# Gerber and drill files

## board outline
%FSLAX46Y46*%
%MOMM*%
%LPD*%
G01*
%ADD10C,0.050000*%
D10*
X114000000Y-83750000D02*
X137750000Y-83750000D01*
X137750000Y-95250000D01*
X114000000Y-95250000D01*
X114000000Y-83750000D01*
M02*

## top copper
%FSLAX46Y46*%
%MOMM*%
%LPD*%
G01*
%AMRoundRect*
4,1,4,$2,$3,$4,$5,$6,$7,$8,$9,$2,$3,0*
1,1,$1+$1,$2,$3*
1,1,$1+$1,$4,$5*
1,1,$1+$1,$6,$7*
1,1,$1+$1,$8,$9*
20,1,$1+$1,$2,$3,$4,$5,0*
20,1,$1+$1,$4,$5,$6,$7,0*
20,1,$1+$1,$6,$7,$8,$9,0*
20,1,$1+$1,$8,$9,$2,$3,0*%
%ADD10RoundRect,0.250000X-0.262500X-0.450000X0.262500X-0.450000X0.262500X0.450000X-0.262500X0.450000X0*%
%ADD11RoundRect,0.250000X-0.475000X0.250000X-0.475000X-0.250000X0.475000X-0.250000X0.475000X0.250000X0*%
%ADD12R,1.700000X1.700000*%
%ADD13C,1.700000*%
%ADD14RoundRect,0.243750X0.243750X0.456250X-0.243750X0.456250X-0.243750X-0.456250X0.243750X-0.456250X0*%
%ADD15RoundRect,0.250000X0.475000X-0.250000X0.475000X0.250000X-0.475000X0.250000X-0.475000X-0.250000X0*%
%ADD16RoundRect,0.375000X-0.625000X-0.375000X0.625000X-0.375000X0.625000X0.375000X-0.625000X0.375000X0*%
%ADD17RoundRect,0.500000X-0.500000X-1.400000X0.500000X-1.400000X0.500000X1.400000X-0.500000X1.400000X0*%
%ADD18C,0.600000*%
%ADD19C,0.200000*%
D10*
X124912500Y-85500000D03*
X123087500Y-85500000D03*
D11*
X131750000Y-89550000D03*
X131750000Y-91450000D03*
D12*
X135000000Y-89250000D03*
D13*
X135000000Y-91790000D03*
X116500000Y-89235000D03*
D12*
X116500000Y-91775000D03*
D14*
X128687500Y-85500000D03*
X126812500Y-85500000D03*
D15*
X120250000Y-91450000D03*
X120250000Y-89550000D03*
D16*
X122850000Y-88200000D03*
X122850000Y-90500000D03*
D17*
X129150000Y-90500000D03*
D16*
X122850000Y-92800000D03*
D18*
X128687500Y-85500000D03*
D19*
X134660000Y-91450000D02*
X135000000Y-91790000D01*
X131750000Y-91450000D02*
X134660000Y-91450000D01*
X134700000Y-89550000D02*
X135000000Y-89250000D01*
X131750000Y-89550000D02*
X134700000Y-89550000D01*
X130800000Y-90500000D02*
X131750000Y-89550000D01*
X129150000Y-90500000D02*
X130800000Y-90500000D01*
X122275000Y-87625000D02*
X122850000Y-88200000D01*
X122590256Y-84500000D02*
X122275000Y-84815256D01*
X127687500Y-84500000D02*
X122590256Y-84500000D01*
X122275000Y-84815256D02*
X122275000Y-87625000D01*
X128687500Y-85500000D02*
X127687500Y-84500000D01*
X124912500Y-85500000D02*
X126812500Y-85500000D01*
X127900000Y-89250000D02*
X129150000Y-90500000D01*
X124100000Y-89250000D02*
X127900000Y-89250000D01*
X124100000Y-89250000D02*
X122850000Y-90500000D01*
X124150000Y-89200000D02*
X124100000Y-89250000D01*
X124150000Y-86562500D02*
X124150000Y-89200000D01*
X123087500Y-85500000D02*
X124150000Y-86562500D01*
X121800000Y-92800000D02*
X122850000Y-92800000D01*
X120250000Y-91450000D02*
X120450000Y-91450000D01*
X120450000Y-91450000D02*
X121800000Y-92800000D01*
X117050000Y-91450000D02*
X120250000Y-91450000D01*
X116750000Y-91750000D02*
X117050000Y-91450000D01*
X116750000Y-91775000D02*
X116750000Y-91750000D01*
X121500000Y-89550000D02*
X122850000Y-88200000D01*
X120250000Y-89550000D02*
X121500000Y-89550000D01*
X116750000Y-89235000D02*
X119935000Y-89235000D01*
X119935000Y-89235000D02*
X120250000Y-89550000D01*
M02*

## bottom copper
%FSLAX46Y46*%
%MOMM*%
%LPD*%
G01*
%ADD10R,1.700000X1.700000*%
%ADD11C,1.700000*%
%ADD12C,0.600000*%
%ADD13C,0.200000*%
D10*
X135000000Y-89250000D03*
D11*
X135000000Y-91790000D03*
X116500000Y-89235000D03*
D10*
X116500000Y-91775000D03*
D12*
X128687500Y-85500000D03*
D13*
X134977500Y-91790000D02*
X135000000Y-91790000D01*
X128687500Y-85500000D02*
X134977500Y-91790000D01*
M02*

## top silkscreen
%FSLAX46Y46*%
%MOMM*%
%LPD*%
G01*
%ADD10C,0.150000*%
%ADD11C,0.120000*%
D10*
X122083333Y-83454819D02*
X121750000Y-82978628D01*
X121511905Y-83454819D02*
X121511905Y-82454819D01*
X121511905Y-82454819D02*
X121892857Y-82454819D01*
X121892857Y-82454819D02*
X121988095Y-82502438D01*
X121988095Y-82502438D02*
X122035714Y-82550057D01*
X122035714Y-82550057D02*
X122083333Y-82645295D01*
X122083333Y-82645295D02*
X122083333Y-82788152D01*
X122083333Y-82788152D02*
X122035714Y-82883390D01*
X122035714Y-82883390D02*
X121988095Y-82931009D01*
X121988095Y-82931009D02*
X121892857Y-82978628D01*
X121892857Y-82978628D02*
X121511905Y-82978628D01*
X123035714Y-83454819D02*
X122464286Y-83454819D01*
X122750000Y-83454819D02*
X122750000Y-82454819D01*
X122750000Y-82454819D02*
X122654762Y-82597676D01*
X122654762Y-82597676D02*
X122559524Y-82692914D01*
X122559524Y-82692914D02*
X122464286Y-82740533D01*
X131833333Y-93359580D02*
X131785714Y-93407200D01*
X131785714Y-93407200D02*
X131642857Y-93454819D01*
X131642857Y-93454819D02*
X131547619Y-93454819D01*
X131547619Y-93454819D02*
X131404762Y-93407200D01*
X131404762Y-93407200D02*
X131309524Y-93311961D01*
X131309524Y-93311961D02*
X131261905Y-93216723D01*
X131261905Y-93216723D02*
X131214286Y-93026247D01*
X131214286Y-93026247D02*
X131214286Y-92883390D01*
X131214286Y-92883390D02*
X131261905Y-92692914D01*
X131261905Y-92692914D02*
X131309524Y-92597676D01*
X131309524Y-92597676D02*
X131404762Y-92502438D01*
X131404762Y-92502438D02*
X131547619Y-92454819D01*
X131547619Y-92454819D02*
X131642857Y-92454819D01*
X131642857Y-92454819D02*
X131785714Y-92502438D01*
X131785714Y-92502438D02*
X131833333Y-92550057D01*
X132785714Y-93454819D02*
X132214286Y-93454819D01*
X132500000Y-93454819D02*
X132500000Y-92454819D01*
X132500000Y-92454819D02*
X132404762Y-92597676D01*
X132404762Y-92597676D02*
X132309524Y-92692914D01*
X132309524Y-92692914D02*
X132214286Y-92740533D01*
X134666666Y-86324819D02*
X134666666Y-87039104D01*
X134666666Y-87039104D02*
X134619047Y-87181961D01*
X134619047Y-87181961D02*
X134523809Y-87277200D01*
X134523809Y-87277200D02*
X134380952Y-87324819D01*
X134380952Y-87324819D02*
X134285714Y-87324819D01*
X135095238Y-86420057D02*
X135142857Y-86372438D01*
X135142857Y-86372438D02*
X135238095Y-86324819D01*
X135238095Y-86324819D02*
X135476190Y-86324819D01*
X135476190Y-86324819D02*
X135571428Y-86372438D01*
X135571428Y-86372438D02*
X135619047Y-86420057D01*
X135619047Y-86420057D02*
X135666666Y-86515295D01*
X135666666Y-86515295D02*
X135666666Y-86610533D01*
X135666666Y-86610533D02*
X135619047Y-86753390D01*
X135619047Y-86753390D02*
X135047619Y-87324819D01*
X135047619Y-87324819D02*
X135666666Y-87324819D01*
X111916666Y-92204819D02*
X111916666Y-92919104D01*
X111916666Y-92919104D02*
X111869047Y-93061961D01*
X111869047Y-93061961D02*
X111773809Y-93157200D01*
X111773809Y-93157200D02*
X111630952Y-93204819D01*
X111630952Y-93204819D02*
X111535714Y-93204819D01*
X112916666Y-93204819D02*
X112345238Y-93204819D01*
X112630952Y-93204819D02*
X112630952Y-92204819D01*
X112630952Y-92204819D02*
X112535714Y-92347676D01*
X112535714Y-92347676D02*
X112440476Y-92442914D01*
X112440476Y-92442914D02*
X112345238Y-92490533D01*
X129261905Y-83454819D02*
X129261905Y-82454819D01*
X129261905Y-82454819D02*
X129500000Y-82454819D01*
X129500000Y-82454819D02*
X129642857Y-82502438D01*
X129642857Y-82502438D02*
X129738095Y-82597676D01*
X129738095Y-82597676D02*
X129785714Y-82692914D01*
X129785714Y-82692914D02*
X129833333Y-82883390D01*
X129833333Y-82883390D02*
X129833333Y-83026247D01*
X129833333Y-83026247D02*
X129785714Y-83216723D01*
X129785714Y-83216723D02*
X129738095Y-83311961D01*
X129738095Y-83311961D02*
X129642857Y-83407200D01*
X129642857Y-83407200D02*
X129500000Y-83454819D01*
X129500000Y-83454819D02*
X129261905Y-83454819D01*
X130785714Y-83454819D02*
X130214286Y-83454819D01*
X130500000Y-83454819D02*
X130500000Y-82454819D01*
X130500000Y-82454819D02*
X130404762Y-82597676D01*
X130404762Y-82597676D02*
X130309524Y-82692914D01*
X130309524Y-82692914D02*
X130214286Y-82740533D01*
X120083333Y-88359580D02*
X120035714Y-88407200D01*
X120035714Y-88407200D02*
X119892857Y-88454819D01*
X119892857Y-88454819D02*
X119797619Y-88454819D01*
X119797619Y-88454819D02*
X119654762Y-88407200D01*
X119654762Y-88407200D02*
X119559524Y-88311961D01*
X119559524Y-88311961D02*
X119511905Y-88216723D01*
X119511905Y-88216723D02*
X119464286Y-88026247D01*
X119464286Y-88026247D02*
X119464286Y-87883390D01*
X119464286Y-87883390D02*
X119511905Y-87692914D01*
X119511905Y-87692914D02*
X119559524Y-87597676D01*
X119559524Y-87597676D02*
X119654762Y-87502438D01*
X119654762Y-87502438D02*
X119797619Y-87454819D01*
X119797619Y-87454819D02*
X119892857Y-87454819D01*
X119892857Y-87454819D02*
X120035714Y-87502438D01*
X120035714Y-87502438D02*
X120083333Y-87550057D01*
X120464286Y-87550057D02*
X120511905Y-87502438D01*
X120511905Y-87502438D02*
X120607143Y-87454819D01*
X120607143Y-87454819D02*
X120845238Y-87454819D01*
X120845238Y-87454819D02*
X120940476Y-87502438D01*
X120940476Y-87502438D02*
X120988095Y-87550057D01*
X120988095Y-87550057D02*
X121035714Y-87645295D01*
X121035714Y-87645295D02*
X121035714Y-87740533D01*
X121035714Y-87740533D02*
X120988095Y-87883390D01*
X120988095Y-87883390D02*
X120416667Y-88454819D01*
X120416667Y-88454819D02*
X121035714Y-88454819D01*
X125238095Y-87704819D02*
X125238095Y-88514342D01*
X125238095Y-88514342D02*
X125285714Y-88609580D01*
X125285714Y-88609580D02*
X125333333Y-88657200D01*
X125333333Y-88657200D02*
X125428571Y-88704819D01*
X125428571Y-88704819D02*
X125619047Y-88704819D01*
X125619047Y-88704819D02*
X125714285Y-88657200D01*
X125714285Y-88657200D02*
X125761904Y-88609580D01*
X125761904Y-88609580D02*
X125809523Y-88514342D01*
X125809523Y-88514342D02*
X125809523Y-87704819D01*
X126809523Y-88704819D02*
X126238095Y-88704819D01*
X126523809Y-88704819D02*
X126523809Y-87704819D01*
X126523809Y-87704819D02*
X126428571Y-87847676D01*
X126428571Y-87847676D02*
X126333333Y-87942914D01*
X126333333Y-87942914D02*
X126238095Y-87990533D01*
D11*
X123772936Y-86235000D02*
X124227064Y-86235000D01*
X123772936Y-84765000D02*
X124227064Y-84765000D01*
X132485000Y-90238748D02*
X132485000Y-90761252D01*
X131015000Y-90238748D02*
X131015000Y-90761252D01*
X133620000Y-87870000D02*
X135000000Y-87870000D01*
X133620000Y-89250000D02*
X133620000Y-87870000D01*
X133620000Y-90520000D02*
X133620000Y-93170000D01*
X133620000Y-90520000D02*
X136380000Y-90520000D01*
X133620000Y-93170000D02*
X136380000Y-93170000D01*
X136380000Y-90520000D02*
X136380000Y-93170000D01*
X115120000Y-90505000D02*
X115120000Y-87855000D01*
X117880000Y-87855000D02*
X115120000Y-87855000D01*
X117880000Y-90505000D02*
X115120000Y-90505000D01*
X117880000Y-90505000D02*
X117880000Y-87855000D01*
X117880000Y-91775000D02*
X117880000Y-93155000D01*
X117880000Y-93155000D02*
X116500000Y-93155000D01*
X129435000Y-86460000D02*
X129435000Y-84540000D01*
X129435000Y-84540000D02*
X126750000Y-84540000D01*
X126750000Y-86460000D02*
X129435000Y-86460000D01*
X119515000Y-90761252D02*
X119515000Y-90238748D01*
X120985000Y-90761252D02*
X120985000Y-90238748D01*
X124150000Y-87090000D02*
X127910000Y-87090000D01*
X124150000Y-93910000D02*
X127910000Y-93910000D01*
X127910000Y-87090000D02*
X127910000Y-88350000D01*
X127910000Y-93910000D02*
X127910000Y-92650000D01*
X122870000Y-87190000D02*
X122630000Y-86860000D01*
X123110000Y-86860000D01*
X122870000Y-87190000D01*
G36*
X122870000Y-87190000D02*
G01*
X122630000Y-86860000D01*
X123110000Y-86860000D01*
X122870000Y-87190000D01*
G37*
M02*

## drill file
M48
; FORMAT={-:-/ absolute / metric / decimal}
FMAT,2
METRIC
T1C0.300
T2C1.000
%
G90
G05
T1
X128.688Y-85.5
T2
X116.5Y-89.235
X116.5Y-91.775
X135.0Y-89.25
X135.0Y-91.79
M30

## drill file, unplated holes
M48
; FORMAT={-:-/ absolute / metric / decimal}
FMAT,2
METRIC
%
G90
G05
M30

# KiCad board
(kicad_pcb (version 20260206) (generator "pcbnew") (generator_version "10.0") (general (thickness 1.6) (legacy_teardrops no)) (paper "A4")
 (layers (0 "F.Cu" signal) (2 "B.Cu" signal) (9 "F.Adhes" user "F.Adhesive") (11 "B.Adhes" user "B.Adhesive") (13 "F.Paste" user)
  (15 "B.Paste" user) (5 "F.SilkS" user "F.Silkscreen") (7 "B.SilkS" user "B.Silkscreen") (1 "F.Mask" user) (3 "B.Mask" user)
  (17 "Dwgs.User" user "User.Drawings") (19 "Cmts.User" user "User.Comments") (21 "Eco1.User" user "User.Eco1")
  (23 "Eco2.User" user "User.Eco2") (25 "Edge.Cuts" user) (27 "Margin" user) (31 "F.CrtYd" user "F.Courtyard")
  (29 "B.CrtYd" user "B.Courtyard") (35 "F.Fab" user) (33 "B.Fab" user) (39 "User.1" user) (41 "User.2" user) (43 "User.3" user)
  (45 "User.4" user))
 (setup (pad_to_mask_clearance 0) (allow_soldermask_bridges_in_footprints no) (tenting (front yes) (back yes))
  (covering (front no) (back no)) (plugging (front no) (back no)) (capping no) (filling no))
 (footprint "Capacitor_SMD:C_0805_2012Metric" (layer "F.Cu") (at 131.75 90.5 -90)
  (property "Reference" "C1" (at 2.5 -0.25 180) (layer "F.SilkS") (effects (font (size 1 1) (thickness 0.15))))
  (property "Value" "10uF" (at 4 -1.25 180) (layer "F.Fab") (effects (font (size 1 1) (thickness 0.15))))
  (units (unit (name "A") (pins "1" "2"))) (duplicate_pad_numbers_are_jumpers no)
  (fp_line (start -0.261252 0.735) (end 0.261252 0.735) (stroke (width 0.12) (type solid)) (layer "F.SilkS"))
  (fp_line (start -0.261252 -0.735) (end 0.261252 -0.735) (stroke (width 0.12) (type solid)) (layer "F.SilkS"))
  (pad "1" smd roundrect (at -0.95 0 270) (size 1 1.45) (layers "F.Cu" "F.Mask" "F.Paste") (roundrect_rratio 0.25) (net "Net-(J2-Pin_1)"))
  (pad "2" smd roundrect (at 0.95 0 270) (size 1 1.45) (layers "F.Cu" "F.Mask" "F.Paste") (roundrect_rratio 0.25) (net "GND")))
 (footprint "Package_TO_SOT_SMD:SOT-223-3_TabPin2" (layer "F.Cu") (at 126 90.5)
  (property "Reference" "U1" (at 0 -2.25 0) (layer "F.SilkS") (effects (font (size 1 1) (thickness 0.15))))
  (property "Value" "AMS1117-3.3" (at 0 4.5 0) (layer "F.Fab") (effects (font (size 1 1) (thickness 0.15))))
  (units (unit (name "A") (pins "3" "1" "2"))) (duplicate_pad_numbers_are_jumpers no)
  (fp_line (start -1.85 -3.41) (end 1.91 -3.41) (stroke (width 0.12) (type solid)) (layer "F.SilkS"))
  (fp_line (start -1.85 3.41) (end 1.91 3.41) (stroke (width 0.12) (type solid)) (layer "F.SilkS"))
  (fp_line (start 1.91 -3.41) (end 1.91 -2.15) (stroke (width 0.12) (type solid)) (layer "F.SilkS"))
  (fp_line (start 1.91 3.41) (end 1.91 2.15) (stroke (width 0.12) (type solid)) (layer "F.SilkS"))
  (fp_poly
   (pts (xy -3.13 -3.31) (xy -3.37 -3.64) (xy -2.89 -3.64) (xy -3.13 -3.31)) (stroke (width 0.12) (type solid)) (fill yes) (layer "F.SilkS"))
  (pad "1" smd roundrect (at -3.15 -2.3) (size 2 1.5) (layers "F.Cu" "F.Mask" "F.Paste") (roundrect_rratio 0.25) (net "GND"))
  (pad "2" smd roundrect (at -3.15 0) (size 2 1.5) (layers "F.Cu" "F.Mask" "F.Paste") (roundrect_rratio 0.25) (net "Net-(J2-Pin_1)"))
  (pad "2" smd roundrect (at 3.15 0) (size 2 3.8) (layers "F.Cu" "F.Mask" "F.Paste") (roundrect_rratio 0.25) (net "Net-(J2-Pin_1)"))
  (pad "3" smd roundrect (at -3.15 2.3) (size 2 1.5) (layers "F.Cu" "F.Mask" "F.Paste") (roundrect_rratio 0.25) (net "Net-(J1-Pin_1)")))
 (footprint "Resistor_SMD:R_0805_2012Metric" (layer "F.Cu") (at 124 85.5)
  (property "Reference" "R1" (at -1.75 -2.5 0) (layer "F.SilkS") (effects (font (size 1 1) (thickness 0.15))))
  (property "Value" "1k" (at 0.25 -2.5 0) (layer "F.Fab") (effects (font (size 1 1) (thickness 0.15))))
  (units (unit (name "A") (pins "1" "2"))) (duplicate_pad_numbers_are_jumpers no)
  (fp_line (start -0.227064 -0.735) (end 0.227064 -0.735) (stroke (width 0.12) (type solid)) (layer "F.SilkS"))
  (fp_line (start -0.227064 0.735) (end 0.227064 0.735) (stroke (width 0.12) (type solid)) (layer "F.SilkS"))
  (pad "1" smd roundrect (at -0.9125 0) (size 1.025 1.4) (layers "F.Cu" "F.Mask" "F.Paste") (roundrect_rratio 0.243902)
   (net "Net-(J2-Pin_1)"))
  (pad "2" smd roundrect (at 0.9125 0) (size 1.025 1.4) (layers "F.Cu" "F.Mask" "F.Paste") (roundrect_rratio 0.243902) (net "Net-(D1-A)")))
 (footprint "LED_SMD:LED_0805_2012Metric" (layer "F.Cu") (at 127.75 85.5 180)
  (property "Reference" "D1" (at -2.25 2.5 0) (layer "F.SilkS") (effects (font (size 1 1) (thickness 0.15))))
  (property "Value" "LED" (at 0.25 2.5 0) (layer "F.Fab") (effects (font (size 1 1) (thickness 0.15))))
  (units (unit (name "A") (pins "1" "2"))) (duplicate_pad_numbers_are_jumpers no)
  (fp_line (start 1 -0.96) (end -1.685 -0.96) (stroke (width 0.12) (type solid)) (layer "F.SilkS"))
  (fp_line (start -1.685 0.96) (end 1 0.96) (stroke (width 0.12) (type solid)) (layer "F.SilkS"))
  (fp_line (start -1.685 -0.96) (end -1.685 0.96) (stroke (width 0.12) (type solid)) (layer "F.SilkS"))
  (pad "1" smd roundrect (at -0.9375 0 180) (size 0.975 1.4) (layers "F.Cu" "F.Mask" "F.Paste") (roundrect_rratio 0.25) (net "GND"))
  (pad "2" smd roundrect (at 0.9375 0 180) (size 0.975 1.4) (layers "F.Cu" "F.Mask" "F.Paste") (roundrect_rratio 0.25) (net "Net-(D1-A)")))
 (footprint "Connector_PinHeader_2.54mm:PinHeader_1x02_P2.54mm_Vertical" (layer "F.Cu") (at 116.5 91.775 180)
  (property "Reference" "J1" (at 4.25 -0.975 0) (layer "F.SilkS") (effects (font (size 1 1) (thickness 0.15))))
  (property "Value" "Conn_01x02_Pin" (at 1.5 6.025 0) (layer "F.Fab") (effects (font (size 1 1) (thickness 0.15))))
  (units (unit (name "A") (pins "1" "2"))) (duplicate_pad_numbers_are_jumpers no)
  (fp_line (start 1.38 1.27) (end 1.38 3.92) (stroke (width 0.12) (type solid)) (layer "F.SilkS"))
  (fp_line (start -1.38 3.92) (end 1.38 3.92) (stroke (width 0.12) (type solid)) (layer "F.SilkS"))
  (fp_line (start -1.38 1.27) (end 1.38 1.27) (stroke (width 0.12) (type solid)) (layer "F.SilkS"))
  (fp_line (start -1.38 1.27) (end -1.38 3.92) (stroke (width 0.12) (type solid)) (layer "F.SilkS"))
  (fp_line (start -1.38 0) (end -1.38 -1.38) (stroke (width 0.12) (type solid)) (layer "F.SilkS"))
  (fp_line (start -1.38 -1.38) (end 0 -1.38) (stroke (width 0.12) (type solid)) (layer "F.SilkS"))
  (pad "1" thru_hole rect (at 0 0 180) (size 1.7 1.7) (drill 1) (layers "*.Cu" "*.Mask") (remove_unused_layers no) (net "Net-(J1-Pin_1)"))
  (pad "2" thru_hole circle (at 0 2.54 180) (size 1.7 1.7) (drill 1) (layers "*.Cu" "*.Mask") (remove_unused_layers no) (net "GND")))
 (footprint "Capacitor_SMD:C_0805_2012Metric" (layer "F.Cu") (at 120.25 90.5 90)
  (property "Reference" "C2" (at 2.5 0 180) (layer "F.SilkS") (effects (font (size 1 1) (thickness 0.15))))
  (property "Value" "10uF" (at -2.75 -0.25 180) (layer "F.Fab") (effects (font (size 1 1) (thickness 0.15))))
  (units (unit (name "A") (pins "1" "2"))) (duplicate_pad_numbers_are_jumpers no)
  (fp_line (start -0.261252 -0.735) (end 0.261252 -0.735) (stroke (width 0.12) (type solid)) (layer "F.SilkS"))
  (fp_line (start -0.261252 0.735) (end 0.261252 0.735) (stroke (width 0.12) (type solid)) (layer "F.SilkS"))
  (pad "1" smd roundrect (at -0.95 0 90) (size 1 1.45) (layers "F.Cu" "F.Mask" "F.Paste") (roundrect_rratio 0.25) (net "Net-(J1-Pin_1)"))
  (pad "2" smd roundrect (at 0.95 0 90) (size 1 1.45) (layers "F.Cu" "F.Mask" "F.Paste") (roundrect_rratio 0.25) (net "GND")))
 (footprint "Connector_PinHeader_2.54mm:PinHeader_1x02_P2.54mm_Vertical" (layer "F.Cu") (at 135 89.25)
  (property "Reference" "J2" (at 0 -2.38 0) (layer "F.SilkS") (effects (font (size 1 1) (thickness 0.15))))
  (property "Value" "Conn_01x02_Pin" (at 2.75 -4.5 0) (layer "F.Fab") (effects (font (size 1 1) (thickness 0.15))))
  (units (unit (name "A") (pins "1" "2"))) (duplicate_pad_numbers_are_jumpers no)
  (fp_line (start -1.38 -1.38) (end 0 -1.38) (stroke (width 0.12) (type solid)) (layer "F.SilkS"))
  (fp_line (start -1.38 0) (end -1.38 -1.38) (stroke (width 0.12) (type solid)) (layer "F.SilkS"))
  (fp_line (start -1.38 1.27) (end -1.38 3.92) (stroke (width 0.12) (type solid)) (layer "F.SilkS"))
  (fp_line (start -1.38 1.27) (end 1.38 1.27) (stroke (width 0.12) (type solid)) (layer "F.SilkS"))
  (fp_line (start -1.38 3.92) (end 1.38 3.92) (stroke (width 0.12) (type solid)) (layer "F.SilkS"))
  (fp_line (start 1.38 1.27) (end 1.38 3.92) (stroke (width 0.12) (type solid)) (layer "F.SilkS"))
  (pad "1" thru_hole rect (at 0 0) (size 1.7 1.7) (drill 1) (layers "*.Cu" "*.Mask") (remove_unused_layers no) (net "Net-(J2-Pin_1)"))
  (pad "2" thru_hole circle (at 0 2.54) (size 1.7 1.7) (drill 1) (layers "*.Cu" "*.Mask") (remove_unused_layers no) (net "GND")))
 (gr_rect (start 114 83.75) (end 137.75 95.25) (stroke (width 0.05) (type default)) (fill no) (layer "Edge.Cuts"))
 (segment (start 124.15 89.2) (end 124.1 89.25) (width 0.2) (layer "F.Cu") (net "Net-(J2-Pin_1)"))
 (segment (start 124.15 86.5625) (end 124.15 89.2) (width 0.2) (layer "F.Cu") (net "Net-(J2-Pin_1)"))
 (segment (start 130.8 90.5) (end 131.75 89.55) (width 0.2) (layer "F.Cu") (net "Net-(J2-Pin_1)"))
 (segment (start 134.7 89.55) (end 135 89.25) (width 0.2) (layer "F.Cu") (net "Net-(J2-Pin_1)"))
 (segment (start 123.0875 85.5) (end 124.15 86.5625) (width 0.2) (layer "F.Cu") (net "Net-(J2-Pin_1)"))
 (segment (start 131.75 89.55) (end 134.7 89.55) (width 0.2) (layer "F.Cu") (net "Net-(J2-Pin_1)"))
 (segment (start 124.1 89.25) (end 122.85 90.5) (width 0.2) (layer "F.Cu") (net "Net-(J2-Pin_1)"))
 (segment (start 124.1 89.25) (end 127.9 89.25) (width 0.2) (layer "F.Cu") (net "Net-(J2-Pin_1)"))
 (segment (start 127.9 89.25) (end 129.15 90.5) (width 0.2) (layer "F.Cu") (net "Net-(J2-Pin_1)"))
 (segment (start 129.15 90.5) (end 130.8 90.5) (width 0.2) (layer "F.Cu") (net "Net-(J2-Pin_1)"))
 (segment (start 119.935 89.235) (end 120.25 89.55) (width 0.2) (layer "F.Cu") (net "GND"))
 (segment (start 116.75 89.235) (end 119.935 89.235) (width 0.2) (layer "F.Cu") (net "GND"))
 (segment (start 121.5 89.55) (end 122.85 88.2) (width 0.2) (layer "F.Cu") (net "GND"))
 (segment (start 122.275 84.815256) (end 122.275 87.625) (width 0.2) (layer "F.Cu") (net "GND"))
 (segment (start 131.75 91.45) (end 134.66 91.45) (width 0.2) (layer "F.Cu") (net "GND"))
 (segment (start 127.6875 84.5) (end 122.590256 84.5) (width 0.2) (layer "F.Cu") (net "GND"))
 (segment (start 122.590256 84.5) (end 122.275 84.815256) (width 0.2) (layer "F.Cu") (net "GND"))
 (segment (start 120.25 89.55) (end 121.5 89.55) (width 0.2) (layer "F.Cu") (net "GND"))
 (segment (start 128.6875 85.5) (end 127.6875 84.5) (width 0.2) (layer "F.Cu") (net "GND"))
 (segment (start 122.275 87.625) (end 122.85 88.2) (width 0.2) (layer "F.Cu") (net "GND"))
 (segment (start 134.66 91.45) (end 135 91.79) (width 0.2) (layer "F.Cu") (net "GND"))
 (via (at 128.6875 85.5) (size 0.6) (drill 0.3) (layers "F.Cu" "B.Cu") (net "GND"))
 (segment (start 128.6875 85.5) (end 134.9775 91.79) (width 0.2) (layer "B.Cu") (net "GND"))
 (segment (start 134.9775 91.79) (end 135 91.79) (width 0.2) (layer "B.Cu") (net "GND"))
 (segment (start 117.05 91.45) (end 120.25 91.45) (width 0.2) (layer "F.Cu") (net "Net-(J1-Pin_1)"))
 (segment (start 120.45 91.45) (end 121.8 92.8) (width 0.2) (layer "F.Cu") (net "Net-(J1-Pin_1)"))
 (segment (start 120.25 91.45) (end 120.45 91.45) (width 0.2) (layer "F.Cu") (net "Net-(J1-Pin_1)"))
 (segment (start 116.75 91.75) (end 117.05 91.45) (width 0.2) (layer "F.Cu") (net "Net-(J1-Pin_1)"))
 (segment (start 116.75 91.775) (end 116.75 91.75) (width 0.2) (layer "F.Cu") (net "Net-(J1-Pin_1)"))
 (segment (start 121.8 92.8) (end 122.85 92.8) (width 0.2) (layer "F.Cu") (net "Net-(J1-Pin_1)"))
 (segment (start 124.9125 85.5) (end 126.8125 85.5) (width 0.2) (layer "F.Cu") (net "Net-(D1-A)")))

